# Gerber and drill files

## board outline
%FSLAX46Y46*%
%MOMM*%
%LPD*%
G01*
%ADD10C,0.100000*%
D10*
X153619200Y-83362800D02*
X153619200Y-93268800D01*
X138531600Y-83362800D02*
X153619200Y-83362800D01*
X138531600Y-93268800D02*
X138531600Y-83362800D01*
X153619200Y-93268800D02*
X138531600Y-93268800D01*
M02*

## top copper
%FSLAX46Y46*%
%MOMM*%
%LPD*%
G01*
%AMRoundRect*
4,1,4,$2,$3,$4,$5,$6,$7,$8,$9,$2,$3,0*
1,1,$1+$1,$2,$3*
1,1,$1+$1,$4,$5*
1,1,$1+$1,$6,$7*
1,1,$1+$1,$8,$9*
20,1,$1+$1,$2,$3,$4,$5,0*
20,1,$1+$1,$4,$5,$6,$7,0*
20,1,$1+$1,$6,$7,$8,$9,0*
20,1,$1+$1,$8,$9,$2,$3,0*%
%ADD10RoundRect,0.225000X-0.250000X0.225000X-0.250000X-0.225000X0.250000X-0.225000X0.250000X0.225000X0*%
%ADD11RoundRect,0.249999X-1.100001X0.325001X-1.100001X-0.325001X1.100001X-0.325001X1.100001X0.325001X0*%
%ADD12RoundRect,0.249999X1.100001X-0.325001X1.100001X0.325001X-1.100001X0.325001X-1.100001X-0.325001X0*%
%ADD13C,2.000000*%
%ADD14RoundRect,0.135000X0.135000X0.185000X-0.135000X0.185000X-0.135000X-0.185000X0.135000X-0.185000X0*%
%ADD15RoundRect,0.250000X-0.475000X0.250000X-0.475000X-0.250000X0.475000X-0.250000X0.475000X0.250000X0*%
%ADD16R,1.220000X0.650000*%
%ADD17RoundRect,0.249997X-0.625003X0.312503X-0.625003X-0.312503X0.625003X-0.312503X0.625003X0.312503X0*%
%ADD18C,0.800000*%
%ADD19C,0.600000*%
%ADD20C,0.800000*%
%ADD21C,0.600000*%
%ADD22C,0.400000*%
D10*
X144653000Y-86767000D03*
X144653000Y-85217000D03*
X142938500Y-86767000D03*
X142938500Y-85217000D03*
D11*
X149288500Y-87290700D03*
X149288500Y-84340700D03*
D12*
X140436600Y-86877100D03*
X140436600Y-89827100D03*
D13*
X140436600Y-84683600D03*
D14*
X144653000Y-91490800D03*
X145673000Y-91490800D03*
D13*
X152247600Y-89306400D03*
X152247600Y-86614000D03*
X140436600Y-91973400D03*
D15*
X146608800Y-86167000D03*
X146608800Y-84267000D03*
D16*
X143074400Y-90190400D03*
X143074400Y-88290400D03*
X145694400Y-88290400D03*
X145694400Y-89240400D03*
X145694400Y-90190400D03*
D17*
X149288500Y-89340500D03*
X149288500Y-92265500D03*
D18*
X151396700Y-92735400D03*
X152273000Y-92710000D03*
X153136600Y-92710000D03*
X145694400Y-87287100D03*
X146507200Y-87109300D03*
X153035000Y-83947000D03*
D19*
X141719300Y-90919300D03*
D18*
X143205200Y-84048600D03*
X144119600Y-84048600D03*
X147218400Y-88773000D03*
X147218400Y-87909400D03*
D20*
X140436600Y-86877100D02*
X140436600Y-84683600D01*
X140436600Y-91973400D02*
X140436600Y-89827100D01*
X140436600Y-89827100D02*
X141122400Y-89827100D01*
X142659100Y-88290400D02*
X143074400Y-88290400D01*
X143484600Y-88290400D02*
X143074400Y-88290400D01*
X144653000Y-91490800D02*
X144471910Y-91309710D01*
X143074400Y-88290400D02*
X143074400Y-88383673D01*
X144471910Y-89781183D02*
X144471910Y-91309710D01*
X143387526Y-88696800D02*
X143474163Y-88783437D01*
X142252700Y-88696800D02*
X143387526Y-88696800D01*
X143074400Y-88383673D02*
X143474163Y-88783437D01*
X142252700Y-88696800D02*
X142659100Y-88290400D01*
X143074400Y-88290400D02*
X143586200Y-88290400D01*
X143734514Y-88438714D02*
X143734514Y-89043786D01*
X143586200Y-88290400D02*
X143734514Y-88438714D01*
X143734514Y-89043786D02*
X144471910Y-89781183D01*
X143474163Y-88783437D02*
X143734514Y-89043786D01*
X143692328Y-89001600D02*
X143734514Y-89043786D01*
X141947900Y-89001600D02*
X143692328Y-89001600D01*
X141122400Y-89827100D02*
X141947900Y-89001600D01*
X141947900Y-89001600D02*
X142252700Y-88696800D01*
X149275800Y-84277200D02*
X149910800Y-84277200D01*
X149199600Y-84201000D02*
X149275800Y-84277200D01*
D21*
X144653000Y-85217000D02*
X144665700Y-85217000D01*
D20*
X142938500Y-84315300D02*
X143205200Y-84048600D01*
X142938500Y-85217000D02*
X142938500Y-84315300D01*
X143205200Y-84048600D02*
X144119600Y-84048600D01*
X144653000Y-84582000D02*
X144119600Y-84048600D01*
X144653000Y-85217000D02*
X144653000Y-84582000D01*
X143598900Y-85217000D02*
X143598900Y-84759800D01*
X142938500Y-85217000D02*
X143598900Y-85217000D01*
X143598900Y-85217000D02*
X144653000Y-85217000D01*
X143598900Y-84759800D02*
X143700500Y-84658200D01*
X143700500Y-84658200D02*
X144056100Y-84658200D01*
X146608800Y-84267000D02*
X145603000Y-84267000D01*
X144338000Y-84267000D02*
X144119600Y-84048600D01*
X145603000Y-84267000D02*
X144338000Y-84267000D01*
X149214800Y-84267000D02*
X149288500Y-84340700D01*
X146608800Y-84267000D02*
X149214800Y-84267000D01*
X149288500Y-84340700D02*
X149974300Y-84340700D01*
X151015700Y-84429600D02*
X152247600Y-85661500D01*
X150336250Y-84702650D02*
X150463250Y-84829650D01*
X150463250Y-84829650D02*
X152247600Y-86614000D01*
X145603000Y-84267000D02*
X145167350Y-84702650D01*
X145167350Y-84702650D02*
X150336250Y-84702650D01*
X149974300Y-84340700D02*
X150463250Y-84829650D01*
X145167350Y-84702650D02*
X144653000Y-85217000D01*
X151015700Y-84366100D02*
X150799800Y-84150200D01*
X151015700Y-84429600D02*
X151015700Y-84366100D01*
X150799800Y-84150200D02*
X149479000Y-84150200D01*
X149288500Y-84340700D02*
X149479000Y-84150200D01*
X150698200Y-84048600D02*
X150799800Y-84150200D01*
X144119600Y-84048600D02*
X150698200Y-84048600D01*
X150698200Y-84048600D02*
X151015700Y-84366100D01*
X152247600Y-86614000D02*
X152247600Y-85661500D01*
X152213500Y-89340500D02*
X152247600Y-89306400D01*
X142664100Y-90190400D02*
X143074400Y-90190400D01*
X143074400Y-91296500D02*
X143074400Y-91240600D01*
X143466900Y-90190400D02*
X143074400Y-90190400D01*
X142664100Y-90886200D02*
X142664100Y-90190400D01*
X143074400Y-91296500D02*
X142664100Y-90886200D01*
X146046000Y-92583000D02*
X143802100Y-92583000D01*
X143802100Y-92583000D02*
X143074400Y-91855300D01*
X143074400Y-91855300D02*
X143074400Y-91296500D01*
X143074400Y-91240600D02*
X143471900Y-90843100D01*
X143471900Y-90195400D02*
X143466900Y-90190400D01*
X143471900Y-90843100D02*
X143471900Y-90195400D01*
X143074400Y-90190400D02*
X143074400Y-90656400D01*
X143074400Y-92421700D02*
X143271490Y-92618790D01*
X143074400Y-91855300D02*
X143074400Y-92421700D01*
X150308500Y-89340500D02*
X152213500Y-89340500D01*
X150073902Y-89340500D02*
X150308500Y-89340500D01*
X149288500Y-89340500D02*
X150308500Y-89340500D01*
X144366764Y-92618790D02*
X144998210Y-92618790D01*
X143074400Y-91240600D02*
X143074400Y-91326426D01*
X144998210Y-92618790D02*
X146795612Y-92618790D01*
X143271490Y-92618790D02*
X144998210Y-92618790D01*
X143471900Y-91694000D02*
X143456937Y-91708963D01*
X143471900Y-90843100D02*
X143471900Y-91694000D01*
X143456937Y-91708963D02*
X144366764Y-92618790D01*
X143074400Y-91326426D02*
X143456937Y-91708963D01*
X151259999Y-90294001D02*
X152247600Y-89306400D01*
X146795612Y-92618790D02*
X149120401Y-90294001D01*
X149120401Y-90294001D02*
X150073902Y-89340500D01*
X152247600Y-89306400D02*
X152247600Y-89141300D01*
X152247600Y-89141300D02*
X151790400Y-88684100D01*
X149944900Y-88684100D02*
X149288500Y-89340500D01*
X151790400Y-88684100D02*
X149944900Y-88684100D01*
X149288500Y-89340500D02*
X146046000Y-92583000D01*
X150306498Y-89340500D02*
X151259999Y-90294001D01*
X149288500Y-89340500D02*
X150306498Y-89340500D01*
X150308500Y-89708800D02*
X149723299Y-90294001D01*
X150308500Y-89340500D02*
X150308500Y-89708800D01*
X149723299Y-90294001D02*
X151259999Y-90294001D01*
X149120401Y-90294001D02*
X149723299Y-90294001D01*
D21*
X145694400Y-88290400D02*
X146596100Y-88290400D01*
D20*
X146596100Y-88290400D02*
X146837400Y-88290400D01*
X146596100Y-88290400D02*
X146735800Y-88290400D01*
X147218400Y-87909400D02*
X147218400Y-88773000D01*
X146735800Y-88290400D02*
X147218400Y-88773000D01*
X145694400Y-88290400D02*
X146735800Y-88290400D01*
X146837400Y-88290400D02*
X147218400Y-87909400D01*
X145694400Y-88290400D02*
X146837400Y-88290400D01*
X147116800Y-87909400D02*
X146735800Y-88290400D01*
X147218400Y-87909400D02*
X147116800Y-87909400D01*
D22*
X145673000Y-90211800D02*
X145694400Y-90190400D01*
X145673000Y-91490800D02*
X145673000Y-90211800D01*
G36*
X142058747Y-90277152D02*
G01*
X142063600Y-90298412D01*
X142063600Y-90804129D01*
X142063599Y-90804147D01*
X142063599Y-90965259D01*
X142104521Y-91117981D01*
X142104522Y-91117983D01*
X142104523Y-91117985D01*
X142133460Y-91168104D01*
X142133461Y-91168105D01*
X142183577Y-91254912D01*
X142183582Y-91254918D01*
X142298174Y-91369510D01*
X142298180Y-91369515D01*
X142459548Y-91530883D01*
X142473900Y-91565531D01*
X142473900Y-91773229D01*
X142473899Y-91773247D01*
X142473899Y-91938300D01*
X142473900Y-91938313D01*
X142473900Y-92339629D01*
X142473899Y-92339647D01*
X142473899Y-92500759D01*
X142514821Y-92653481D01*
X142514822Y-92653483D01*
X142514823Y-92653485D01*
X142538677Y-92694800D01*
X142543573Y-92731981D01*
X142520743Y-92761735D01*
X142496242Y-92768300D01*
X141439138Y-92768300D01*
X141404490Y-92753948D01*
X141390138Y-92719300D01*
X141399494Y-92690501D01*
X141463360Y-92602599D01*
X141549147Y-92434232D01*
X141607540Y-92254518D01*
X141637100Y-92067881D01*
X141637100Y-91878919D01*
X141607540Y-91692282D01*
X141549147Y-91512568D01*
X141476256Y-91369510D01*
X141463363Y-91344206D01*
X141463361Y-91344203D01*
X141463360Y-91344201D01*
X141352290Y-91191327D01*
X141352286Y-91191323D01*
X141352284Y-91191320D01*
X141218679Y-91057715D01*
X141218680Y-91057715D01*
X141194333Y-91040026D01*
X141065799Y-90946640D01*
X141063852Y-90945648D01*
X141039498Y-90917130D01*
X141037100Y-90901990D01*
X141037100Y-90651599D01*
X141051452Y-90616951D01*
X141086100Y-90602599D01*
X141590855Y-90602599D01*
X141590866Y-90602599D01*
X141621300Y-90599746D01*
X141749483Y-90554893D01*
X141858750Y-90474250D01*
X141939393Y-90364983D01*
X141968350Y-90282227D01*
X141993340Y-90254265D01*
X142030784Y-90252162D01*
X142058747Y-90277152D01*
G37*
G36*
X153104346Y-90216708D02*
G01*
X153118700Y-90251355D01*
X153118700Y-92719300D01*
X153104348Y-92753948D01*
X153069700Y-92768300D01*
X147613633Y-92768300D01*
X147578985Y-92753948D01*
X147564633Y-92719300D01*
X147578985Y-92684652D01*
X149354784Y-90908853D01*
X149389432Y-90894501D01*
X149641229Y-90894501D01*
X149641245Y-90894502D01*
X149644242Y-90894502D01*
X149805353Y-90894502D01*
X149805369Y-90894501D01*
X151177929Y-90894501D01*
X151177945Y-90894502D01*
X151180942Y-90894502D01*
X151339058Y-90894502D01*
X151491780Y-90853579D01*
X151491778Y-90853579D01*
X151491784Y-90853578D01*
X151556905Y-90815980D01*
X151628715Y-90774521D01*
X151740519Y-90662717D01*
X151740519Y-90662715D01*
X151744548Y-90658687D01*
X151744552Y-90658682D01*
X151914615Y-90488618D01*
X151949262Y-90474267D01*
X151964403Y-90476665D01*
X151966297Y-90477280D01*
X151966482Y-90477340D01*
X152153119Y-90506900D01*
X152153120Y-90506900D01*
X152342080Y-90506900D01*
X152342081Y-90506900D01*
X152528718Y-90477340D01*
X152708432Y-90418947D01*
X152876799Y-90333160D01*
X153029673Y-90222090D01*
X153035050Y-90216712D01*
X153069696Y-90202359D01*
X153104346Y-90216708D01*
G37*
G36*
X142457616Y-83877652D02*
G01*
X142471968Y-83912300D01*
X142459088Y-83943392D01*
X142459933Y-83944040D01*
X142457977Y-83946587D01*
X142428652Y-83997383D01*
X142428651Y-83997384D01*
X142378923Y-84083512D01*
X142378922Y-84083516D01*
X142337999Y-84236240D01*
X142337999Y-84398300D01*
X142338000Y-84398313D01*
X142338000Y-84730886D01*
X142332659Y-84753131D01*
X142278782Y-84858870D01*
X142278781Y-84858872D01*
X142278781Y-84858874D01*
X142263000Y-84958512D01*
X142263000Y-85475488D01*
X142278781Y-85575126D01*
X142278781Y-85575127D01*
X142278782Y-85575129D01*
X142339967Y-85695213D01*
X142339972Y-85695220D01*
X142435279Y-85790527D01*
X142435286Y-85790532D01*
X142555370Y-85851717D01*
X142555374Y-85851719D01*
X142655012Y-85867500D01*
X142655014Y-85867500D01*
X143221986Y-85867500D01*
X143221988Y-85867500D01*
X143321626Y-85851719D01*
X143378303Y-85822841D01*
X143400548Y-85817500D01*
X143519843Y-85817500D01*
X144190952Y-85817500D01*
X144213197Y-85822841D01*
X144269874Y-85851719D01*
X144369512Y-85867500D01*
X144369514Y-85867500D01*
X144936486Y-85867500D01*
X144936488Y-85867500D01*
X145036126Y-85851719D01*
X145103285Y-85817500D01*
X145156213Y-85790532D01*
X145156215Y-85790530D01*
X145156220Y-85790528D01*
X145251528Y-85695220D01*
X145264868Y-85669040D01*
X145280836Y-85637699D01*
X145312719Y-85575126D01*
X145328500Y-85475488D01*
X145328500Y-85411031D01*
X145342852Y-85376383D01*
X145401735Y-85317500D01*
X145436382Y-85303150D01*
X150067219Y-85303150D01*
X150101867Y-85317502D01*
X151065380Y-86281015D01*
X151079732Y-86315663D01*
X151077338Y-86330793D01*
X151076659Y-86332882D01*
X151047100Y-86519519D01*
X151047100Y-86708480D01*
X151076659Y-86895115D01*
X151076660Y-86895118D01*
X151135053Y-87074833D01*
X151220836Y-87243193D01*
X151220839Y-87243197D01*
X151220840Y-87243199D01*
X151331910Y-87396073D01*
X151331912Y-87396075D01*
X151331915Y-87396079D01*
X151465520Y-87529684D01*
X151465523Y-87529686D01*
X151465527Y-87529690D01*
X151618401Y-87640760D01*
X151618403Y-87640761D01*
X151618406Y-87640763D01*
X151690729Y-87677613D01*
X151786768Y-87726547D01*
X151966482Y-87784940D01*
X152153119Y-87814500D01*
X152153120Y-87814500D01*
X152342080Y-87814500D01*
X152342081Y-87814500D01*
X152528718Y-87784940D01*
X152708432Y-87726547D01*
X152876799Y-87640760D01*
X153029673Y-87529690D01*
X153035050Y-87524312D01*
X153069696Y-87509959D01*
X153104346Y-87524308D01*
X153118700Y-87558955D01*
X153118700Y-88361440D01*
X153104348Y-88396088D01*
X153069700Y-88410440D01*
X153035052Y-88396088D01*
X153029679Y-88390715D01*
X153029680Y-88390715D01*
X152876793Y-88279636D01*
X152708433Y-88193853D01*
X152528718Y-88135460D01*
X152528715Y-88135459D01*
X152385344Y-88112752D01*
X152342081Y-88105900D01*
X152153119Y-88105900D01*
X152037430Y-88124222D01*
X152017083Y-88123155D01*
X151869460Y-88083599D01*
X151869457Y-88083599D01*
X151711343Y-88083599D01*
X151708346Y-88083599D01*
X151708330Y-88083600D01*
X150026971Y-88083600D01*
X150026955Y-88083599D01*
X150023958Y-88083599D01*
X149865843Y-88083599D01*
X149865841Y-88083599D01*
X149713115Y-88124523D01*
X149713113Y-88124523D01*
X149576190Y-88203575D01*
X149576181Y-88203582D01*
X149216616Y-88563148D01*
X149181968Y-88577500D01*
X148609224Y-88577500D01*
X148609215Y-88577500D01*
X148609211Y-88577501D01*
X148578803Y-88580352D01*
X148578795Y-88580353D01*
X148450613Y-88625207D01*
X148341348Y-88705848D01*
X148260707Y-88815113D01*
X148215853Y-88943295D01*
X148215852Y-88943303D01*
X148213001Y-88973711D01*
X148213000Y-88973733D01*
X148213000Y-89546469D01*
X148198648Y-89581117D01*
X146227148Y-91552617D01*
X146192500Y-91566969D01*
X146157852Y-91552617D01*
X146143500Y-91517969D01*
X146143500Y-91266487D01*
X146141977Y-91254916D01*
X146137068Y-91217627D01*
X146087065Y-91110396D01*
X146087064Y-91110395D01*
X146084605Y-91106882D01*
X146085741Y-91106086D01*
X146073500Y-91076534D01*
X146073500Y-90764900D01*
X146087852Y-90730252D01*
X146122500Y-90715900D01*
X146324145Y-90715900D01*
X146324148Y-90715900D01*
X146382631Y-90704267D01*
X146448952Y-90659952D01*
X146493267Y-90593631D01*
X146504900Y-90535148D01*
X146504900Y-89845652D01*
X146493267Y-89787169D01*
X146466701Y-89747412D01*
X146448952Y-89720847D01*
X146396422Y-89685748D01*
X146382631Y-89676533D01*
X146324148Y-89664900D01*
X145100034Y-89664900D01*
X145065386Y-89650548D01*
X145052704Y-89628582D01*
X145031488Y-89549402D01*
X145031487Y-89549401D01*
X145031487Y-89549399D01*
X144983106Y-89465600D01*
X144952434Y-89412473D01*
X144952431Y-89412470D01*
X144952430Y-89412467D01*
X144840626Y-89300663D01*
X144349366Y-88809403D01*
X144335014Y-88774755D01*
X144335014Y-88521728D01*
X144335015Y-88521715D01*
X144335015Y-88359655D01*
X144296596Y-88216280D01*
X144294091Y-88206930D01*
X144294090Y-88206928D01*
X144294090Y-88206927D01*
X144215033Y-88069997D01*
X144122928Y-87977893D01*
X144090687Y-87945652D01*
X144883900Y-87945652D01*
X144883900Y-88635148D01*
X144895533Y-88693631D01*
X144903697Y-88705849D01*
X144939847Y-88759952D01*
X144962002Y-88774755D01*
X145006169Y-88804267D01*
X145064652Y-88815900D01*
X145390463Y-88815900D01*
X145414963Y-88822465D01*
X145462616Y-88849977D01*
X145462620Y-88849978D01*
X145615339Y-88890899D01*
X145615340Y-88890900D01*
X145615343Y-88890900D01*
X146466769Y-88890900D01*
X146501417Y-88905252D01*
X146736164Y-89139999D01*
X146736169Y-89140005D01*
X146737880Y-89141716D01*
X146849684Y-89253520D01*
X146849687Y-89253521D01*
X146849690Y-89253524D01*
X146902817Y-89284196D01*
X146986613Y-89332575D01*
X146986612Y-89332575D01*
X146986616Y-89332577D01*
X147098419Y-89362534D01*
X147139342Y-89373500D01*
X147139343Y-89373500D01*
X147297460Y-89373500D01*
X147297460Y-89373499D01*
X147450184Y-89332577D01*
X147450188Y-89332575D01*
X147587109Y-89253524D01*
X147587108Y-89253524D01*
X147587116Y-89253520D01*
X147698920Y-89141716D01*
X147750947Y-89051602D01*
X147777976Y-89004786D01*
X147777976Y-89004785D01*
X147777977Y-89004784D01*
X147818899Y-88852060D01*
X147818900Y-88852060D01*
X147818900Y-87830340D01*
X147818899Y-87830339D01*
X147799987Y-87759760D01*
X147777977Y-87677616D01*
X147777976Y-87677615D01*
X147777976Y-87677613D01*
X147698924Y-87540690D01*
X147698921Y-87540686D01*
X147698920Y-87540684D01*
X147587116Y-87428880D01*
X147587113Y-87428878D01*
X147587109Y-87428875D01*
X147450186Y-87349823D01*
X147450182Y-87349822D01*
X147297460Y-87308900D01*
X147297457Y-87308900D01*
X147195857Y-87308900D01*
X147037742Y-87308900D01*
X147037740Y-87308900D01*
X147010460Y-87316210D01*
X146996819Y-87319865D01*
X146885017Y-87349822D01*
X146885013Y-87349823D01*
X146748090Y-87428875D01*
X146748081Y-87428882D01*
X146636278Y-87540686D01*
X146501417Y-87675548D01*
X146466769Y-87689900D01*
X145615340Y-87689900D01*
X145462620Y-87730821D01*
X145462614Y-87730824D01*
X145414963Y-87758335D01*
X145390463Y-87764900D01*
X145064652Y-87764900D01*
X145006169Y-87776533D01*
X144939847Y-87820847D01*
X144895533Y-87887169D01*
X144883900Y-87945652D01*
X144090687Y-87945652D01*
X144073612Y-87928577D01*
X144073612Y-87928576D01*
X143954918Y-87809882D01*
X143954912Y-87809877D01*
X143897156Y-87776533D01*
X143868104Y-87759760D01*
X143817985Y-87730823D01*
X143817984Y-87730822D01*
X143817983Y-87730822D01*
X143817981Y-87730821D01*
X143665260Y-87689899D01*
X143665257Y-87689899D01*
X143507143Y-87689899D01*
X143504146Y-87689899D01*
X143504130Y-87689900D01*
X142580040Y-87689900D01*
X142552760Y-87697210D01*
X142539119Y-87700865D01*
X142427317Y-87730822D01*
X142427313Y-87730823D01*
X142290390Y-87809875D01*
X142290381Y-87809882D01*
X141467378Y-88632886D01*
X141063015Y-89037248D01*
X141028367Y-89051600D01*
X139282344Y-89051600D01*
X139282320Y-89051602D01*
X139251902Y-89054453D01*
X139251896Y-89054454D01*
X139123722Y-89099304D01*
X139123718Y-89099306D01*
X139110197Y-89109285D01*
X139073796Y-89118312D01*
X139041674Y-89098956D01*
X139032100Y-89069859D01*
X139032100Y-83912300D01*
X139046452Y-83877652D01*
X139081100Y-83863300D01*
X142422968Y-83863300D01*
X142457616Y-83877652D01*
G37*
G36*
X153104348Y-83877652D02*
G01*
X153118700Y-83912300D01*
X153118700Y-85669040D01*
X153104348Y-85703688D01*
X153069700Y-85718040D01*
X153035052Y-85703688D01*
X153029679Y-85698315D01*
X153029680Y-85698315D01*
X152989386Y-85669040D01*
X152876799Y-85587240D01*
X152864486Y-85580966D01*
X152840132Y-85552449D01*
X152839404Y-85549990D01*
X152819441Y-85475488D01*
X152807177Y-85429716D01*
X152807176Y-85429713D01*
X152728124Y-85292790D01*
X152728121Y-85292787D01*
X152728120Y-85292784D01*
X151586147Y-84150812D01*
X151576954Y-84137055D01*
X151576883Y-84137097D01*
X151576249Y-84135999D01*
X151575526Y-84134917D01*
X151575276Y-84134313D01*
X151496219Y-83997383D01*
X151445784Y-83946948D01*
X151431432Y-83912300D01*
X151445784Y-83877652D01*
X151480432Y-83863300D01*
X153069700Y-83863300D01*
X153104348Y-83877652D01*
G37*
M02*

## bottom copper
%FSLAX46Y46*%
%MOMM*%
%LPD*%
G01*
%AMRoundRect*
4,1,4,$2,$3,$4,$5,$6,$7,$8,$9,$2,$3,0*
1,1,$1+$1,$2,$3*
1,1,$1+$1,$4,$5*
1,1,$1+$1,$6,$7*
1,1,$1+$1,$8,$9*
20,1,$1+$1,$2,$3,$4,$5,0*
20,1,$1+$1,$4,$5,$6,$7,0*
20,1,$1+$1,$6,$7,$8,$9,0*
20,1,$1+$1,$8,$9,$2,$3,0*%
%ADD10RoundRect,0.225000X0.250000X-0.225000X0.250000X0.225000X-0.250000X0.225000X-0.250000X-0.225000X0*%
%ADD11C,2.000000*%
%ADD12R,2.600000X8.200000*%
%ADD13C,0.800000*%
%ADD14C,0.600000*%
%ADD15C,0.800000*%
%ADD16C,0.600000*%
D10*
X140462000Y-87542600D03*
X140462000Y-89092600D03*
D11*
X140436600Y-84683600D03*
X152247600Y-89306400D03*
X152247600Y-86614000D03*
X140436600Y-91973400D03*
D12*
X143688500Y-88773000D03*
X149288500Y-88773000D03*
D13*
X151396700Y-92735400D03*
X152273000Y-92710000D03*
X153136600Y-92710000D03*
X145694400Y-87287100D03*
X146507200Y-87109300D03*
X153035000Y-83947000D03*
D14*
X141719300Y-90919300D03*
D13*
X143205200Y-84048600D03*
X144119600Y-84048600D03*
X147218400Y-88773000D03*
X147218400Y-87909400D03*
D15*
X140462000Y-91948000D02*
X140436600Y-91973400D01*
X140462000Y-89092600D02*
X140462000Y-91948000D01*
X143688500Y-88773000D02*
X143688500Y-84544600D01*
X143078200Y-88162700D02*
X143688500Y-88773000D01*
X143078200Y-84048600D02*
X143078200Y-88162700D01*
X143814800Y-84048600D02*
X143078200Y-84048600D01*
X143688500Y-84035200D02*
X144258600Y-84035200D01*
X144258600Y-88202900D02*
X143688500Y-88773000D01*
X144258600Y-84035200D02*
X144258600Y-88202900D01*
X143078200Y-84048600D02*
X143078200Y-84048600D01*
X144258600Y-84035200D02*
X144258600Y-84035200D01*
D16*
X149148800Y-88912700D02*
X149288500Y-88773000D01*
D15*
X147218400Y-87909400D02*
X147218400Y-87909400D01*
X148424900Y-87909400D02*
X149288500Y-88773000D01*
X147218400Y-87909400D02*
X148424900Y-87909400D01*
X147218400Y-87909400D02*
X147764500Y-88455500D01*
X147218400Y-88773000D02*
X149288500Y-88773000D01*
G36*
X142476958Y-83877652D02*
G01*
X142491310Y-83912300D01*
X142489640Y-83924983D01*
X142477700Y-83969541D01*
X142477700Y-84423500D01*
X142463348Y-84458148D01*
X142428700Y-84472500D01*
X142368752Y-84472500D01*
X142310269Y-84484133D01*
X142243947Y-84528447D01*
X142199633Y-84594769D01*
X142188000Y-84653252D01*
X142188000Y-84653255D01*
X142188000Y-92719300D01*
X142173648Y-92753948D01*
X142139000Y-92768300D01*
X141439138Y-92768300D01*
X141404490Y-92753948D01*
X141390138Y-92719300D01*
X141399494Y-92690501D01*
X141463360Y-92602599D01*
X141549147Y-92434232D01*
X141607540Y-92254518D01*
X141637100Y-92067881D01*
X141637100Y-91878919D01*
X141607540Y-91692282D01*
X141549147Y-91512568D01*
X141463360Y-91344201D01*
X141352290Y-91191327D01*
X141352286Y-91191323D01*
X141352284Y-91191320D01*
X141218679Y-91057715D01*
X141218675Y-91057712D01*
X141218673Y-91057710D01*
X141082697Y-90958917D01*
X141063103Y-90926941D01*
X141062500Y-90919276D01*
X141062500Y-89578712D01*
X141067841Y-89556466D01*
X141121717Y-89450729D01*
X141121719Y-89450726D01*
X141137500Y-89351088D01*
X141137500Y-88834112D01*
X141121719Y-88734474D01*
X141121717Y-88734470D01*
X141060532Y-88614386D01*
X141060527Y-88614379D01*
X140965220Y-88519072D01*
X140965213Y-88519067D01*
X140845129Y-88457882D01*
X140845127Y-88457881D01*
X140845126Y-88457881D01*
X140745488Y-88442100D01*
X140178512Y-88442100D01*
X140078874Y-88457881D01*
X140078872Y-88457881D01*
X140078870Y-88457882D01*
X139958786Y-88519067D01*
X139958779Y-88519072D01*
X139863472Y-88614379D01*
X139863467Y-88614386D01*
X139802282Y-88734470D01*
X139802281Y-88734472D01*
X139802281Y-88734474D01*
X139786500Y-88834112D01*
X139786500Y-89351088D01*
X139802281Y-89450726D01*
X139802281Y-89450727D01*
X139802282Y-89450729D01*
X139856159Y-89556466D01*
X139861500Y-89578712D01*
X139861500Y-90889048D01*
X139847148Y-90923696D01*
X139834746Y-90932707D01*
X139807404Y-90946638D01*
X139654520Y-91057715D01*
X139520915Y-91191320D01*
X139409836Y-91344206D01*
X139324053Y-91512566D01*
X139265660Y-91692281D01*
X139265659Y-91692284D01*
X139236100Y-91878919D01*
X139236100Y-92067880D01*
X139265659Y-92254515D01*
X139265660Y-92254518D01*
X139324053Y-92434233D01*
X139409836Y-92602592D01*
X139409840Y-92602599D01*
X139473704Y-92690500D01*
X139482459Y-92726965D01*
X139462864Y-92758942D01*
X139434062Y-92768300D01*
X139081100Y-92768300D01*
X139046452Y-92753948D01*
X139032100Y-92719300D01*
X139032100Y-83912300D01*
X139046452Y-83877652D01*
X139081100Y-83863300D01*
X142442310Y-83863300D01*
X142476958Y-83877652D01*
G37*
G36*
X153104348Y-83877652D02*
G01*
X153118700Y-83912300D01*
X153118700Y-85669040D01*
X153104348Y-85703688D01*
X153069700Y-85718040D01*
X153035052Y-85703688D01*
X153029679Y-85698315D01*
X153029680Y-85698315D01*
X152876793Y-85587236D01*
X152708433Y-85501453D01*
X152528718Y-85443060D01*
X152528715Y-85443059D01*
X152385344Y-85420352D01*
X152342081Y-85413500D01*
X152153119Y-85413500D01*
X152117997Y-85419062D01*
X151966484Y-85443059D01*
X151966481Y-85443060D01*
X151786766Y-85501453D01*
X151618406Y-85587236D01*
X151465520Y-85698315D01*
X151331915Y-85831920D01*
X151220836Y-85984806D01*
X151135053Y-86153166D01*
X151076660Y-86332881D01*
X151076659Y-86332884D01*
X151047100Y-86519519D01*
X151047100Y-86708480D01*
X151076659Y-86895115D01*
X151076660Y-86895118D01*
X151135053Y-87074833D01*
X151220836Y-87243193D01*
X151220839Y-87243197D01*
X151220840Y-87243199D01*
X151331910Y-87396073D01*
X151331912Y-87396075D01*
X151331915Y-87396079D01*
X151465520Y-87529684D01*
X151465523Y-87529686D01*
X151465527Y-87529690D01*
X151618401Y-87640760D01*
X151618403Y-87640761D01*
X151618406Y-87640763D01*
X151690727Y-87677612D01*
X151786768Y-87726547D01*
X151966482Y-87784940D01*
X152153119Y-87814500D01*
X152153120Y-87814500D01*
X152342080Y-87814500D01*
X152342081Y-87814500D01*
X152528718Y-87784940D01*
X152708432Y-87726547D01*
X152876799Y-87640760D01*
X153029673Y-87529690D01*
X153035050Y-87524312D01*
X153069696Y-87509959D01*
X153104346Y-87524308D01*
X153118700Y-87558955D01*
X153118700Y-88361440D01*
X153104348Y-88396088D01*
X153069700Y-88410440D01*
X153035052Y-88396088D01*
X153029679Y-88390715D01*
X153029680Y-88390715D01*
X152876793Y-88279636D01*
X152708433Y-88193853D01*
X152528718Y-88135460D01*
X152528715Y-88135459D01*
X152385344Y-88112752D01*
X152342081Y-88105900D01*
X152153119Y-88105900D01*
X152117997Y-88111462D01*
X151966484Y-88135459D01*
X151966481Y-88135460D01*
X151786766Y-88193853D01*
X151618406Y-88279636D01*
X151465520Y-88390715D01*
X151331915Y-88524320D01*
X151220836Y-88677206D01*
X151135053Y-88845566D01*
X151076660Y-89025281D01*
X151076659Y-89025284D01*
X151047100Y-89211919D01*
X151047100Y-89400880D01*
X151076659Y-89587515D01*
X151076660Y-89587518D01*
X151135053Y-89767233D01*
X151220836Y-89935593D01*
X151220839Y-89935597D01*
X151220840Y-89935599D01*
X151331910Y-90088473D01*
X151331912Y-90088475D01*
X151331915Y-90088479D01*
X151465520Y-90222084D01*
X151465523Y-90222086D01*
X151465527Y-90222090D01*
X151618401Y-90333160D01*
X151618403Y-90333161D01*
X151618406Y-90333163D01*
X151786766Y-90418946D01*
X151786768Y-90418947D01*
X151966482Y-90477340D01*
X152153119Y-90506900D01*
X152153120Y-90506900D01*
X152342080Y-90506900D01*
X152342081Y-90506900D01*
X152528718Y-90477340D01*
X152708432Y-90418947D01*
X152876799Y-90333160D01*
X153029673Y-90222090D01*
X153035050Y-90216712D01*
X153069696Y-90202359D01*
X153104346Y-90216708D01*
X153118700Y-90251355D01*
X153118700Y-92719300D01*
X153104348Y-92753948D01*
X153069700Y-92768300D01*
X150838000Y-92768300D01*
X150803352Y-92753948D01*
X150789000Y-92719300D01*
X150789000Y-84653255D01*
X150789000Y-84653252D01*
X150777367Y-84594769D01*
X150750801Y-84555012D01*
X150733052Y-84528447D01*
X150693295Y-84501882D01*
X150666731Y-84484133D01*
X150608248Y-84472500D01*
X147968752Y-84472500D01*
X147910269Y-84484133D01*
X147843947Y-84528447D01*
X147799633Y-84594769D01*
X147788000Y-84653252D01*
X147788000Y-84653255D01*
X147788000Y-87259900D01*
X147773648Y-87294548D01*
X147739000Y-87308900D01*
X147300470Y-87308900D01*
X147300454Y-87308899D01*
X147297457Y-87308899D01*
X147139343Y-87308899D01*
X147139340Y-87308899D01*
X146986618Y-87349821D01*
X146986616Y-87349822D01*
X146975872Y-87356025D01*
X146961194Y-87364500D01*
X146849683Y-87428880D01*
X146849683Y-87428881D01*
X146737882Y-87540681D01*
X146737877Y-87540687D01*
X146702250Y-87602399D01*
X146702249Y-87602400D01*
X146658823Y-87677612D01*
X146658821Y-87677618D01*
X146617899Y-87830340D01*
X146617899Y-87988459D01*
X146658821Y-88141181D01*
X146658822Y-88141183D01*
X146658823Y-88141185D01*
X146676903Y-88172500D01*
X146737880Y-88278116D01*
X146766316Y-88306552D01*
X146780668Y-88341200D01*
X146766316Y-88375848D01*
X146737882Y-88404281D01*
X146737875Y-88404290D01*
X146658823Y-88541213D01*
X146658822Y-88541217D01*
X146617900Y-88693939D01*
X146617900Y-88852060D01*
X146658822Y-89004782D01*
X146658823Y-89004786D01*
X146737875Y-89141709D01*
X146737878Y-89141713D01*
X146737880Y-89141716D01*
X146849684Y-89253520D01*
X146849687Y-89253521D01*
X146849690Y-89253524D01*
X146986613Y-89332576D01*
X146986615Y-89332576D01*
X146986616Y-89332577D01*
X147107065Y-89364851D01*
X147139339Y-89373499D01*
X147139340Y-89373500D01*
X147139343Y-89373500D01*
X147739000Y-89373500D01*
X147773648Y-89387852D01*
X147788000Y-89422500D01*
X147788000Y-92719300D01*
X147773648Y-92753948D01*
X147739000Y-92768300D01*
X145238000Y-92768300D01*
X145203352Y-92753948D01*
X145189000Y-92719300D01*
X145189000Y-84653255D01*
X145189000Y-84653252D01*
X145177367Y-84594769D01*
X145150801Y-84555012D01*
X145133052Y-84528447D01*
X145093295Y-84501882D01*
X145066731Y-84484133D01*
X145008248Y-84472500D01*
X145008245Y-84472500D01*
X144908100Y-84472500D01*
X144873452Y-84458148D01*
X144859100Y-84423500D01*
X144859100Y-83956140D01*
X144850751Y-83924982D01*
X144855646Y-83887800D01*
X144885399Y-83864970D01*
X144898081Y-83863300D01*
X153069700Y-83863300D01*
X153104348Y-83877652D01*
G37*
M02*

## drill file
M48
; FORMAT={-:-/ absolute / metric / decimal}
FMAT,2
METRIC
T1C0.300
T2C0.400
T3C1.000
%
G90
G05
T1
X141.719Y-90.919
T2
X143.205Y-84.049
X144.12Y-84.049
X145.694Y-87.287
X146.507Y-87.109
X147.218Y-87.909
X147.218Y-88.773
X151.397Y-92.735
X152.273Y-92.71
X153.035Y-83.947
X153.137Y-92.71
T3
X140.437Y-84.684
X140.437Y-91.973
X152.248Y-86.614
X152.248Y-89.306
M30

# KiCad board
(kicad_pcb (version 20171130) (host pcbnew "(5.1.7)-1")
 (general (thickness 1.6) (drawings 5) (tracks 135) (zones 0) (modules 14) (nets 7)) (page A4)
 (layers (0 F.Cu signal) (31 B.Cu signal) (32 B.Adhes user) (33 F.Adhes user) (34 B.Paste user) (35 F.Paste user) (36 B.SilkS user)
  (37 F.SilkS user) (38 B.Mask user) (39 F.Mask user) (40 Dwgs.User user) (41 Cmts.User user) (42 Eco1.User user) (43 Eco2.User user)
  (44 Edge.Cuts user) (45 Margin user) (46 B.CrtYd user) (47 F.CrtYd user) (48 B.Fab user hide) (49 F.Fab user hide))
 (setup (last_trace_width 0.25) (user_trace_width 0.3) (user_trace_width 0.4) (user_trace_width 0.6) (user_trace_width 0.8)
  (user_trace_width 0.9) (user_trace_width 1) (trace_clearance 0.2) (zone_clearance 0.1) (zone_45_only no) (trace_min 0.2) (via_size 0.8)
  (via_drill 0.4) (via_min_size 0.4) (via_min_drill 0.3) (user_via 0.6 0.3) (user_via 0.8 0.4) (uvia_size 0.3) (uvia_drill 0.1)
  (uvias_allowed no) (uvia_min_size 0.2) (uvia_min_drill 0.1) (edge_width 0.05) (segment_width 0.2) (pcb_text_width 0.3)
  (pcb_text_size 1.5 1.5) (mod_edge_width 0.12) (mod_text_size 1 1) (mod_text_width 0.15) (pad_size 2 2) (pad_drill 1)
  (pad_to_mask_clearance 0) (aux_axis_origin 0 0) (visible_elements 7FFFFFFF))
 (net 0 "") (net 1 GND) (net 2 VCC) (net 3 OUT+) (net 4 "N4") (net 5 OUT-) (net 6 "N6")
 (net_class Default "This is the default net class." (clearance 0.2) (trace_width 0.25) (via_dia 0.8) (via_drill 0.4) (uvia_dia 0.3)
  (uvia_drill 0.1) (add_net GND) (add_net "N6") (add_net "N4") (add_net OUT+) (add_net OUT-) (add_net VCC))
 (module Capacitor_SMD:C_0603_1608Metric (layer B.Cu) (at 140.462 88.3176 90)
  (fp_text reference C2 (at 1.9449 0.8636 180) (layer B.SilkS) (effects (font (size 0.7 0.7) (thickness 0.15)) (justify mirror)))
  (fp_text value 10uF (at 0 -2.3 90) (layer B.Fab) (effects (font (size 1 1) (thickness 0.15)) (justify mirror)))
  (pad 2 smd roundrect (at 0.775 0 90) (size 0.9 0.95) (layers B.Cu B.Paste B.Mask) (roundrect_rratio 0.25) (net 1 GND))
  (pad 1 smd roundrect (at -0.775 0 90) (size 0.9 0.95) (layers B.Cu B.Paste B.Mask) (roundrect_rratio 0.25) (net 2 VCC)))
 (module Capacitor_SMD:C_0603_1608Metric (layer F.Cu) (at 144.653 85.992 270)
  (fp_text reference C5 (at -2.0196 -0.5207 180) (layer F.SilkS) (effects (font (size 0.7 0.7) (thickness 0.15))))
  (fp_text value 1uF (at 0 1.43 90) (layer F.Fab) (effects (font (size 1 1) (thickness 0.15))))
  (pad 2 smd roundrect (at 0.775 0 270) (size 0.9 0.95) (layers F.Cu F.Paste F.Mask) (roundrect_rratio 0.25) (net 1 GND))
  (pad 1 smd roundrect (at -0.775 0 270) (size 0.9 0.95) (layers F.Cu F.Paste F.Mask) (roundrect_rratio 0.25) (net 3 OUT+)))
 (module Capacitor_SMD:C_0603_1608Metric (layer F.Cu) (at 142.9385 85.992 270)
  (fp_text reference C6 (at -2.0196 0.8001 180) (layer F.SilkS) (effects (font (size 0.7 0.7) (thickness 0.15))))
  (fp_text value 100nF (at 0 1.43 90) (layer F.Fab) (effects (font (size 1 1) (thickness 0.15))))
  (pad 2 smd roundrect (at 0.775 0 270) (size 0.9 0.95) (layers F.Cu F.Paste F.Mask) (roundrect_rratio 0.25) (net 1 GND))
  (pad 1 smd roundrect (at -0.775 0 270) (size 0.9 0.95) (layers F.Cu F.Paste F.Mask) (roundrect_rratio 0.25) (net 3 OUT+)))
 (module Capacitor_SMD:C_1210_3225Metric (layer F.Cu) (at 149.2885 85.8157 270)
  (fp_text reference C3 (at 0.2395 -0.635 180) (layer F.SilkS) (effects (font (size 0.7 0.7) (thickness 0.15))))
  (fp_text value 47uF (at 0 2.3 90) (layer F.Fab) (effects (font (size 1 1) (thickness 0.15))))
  (pad 2 smd roundrect (at 1.475 0 270) (size 1.15 2.7) (layers F.Cu F.Paste F.Mask) (roundrect_rratio 0.2173904347826087) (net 1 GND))
  (pad 1 smd roundrect (at -1.475 0 270) (size 1.15 2.7) (layers F.Cu F.Paste F.Mask) (roundrect_rratio 0.2173904347826087) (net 3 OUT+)))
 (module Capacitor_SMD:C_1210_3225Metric (layer F.Cu) (at 140.4366 88.3521 90)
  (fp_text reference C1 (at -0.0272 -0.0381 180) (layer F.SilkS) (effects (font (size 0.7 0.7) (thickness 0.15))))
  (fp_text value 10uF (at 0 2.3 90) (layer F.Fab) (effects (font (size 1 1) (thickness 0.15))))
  (pad 2 smd roundrect (at 1.475 0 90) (size 1.15 2.7) (layers F.Cu F.Paste F.Mask) (roundrect_rratio 0.2173904347826087) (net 1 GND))
  (pad 1 smd roundrect (at -1.475 0 90) (size 1.15 2.7) (layers F.Cu F.Paste F.Mask) (roundrect_rratio 0.2173904347826087) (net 2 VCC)))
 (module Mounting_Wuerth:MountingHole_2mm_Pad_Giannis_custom (layer F.Cu) (at 140.4366 84.3661)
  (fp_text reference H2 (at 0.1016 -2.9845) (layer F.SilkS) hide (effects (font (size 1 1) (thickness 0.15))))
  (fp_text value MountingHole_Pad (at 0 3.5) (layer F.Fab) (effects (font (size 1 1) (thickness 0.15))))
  (pad 1 thru_hole circle (at 0 0.3175) (size 2 2) (drill 1) (layers *.Cu *.Mask) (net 1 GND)))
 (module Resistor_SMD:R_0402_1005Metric (layer F.Cu) (at 145.163 91.4908 180)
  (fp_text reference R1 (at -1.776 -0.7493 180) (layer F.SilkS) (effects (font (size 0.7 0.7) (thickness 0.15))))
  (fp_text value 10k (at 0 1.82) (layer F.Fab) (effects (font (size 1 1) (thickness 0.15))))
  (pad 2 smd roundrect (at 0.51 0 180) (size 0.54 0.64) (layers F.Cu F.Paste F.Mask) (roundrect_rratio 0.25) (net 2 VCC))
  (pad 1 smd roundrect (at -0.51 0 180) (size 0.54 0.64) (layers F.Cu F.Paste F.Mask) (roundrect_rratio 0.25) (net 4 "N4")))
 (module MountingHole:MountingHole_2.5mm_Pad (layer F.Cu) (at 154.686 89.408)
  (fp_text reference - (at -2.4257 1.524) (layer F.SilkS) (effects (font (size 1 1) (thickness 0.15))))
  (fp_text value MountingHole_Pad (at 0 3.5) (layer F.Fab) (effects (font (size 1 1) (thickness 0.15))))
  (pad 1 thru_hole circle (at -2.4384 -0.1016) (size 2 2) (drill 1) (layers *.Cu *.Mask) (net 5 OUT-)))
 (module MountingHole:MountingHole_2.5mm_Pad (layer F.Cu) (at 154.686 86.106)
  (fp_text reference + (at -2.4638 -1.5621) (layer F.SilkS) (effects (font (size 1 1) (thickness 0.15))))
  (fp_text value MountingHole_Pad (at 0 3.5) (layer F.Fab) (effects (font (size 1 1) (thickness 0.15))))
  (pad 1 thru_hole circle (at -2.4384 0.508) (size 2 2) (drill 1) (layers *.Cu *.Mask) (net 3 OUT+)))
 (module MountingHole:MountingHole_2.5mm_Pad (layer F.Cu) (at 139.6746 89.8271)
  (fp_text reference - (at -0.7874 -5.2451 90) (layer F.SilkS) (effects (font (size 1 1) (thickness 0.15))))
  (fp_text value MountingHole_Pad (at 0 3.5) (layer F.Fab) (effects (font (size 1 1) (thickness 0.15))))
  (pad 1 thru_hole circle (at 0.762 2.1463) (size 2 2) (drill 1) (layers *.Cu *.Mask) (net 2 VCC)))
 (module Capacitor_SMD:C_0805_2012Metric (layer F.Cu) (at 146.6088 85.217 270)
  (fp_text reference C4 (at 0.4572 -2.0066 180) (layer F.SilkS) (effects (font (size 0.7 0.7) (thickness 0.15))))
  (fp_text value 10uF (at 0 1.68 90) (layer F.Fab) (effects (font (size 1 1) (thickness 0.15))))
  (pad 2 smd roundrect (at 0.95 0 270) (size 1 1.45) (layers F.Cu F.Paste F.Mask) (roundrect_rratio 0.25) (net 1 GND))
  (pad 1 smd roundrect (at -0.95 0 270) (size 1 1.45) (layers F.Cu F.Paste F.Mask) (roundrect_rratio 0.25) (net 3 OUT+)))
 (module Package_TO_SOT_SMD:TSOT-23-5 (layer F.Cu) (at 144.3844 89.2404 180)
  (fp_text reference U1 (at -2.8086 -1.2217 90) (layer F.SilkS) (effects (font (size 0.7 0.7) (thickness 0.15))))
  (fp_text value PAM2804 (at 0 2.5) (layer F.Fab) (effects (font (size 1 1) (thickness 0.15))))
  (pad 5 smd rect (at 1.31 -0.95 180) (size 1.22 0.65) (layers F.Cu F.Paste F.Mask) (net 5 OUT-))
  (pad 4 smd rect (at 1.31 0.95 180) (size 1.22 0.65) (layers F.Cu F.Paste F.Mask) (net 2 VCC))
  (pad 3 smd rect (at -1.31 0.95 180) (size 1.22 0.65) (layers F.Cu F.Paste F.Mask) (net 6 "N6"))
  (pad 2 smd rect (at -1.31 0 180) (size 1.22 0.65) (layers F.Cu F.Paste F.Mask) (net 1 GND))
  (pad 1 smd rect (at -1.31 -0.95 180) (size 1.22 0.65) (layers F.Cu F.Paste F.Mask) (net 4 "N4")))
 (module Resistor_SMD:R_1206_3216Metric (layer F.Cu) (at 149.2885 90.803 270)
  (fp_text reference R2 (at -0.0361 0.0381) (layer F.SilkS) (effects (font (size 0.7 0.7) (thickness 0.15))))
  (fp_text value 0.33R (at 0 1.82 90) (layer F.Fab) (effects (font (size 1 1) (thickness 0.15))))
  (pad 1 smd roundrect (at -1.4625 0 270) (size 1.125 1.75) (layers F.Cu F.Paste F.Mask) (roundrect_rratio 0.2222195555555556) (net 5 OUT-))
  (pad 2 smd roundrect (at 1.4625 0 270) (size 1.125 1.75) (layers F.Cu F.Paste F.Mask) (roundrect_rratio 0.2222195555555556) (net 1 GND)))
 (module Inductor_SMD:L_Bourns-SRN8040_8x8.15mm (layer B.Cu) (at 146.4885 88.773 180)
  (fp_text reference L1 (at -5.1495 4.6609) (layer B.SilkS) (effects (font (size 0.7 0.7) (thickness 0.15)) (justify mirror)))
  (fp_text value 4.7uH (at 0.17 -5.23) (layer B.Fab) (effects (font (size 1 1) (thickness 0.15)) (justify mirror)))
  (pad 2 smd rect (at 2.8 0 180) (size 2.6 8.2) (layers B.Cu B.Paste B.Mask) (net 3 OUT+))
  (pad 1 smd rect (at -2.8 0 180) (size 2.6 8.2) (layers B.Cu B.Paste B.Mask) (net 6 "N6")))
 (gr_line (start 153.6192 83.3628) (end 153.6192 93.2688) (layer Edge.Cuts) (width 0.1))
 (gr_line (start 138.5316 83.3628) (end 153.6192 83.3628) (layer Edge.Cuts) (width 0.1))
 (gr_line (start 138.5316 93.2688) (end 138.5316 83.3628) (layer Edge.Cuts) (width 0.1))
 (gr_line (start 153.6192 93.2688) (end 138.5316 93.2688) (layer Edge.Cuts) (width 0.1))
 (segment (start 140.4366 86.8771) (end 140.4366 84.6836) (width 0.8) (layer F.Cu) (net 1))
 (via (at 151.3967 92.7354) (size 0.8) (drill 0.4) (layers F.Cu B.Cu) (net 1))
 (via (at 152.273 92.71) (size 0.8) (drill 0.4) (layers F.Cu B.Cu) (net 1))
 (via (at 153.1366 92.71) (size 0.8) (drill 0.4) (layers F.Cu B.Cu) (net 1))
 (via (at 145.6944 87.2871) (size 0.8) (drill 0.4) (layers F.Cu B.Cu) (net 1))
 (via (at 146.5072 87.1093) (size 0.8) (drill 0.4) (layers F.Cu B.Cu) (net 1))
 (via (at 153.035 83.947) (size 0.8) (drill 0.4) (layers F.Cu B.Cu) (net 1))
 (via (at 141.7193 90.9193) (size 0.6) (drill 0.3) (layers F.Cu B.Cu) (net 1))
 (segment (start 140.4366 91.9734) (end 140.4366 89.8271) (width 0.8) (layer F.Cu) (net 2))
 (segment (start 140.4366 89.8271) (end 141.1224 89.8271) (width 0.8) (layer F.Cu) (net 2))
 (segment (start 142.6591 88.2904) (end 143.0744 88.2904) (width 0.8) (layer F.Cu) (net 2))
 (segment (start 143.4846 88.2904) (end 143.0744 88.2904) (width 0.8) (layer F.Cu) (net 2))
 (segment (start 144.653 91.4908) (end 144.47191 91.30971) (width 0.8) (layer F.Cu) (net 2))
 (segment (start 143.0744 88.2904) (end 143.0744 88.383673) (width 0.8) (layer F.Cu) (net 2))
 (segment (start 144.47191 89.781183) (end 144.47191 91.30971) (width 0.8) (layer F.Cu) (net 2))
 (segment (start 143.387526 88.6968) (end 143.474163 88.783437) (width 0.8) (layer F.Cu) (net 2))
 (segment (start 142.2527 88.6968) (end 143.387526 88.6968) (width 0.8) (layer F.Cu) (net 2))
 (segment (start 143.0744 88.383673) (end 143.474163 88.783437) (width 0.8) (layer F.Cu) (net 2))
 (segment (start 142.2527 88.6968) (end 142.6591 88.2904) (width 0.8) (layer F.Cu) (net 2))
 (segment (start 143.0744 88.2904) (end 143.5862 88.2904) (width 0.8) (layer F.Cu) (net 2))
 (segment (start 143.734514 88.438714) (end 143.734514 89.043786) (width 0.8) (layer F.Cu) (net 2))
 (segment (start 143.5862 88.2904) (end 143.734514 88.438714) (width 0.8) (layer F.Cu) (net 2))
 (segment (start 143.734514 89.043786) (end 144.47191 89.781183) (width 0.8) (layer F.Cu) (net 2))
 (segment (start 143.474163 88.783437) (end 143.734514 89.043786) (width 0.8) (layer F.Cu) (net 2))
 (segment (start 143.692328 89.0016) (end 143.734514 89.043786) (width 0.8) (layer F.Cu) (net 2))
 (segment (start 141.9479 89.0016) (end 143.692328 89.0016) (width 0.8) (layer F.Cu) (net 2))
 (segment (start 141.1224 89.8271) (end 141.9479 89.0016) (width 0.8) (layer F.Cu) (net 2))
 (segment (start 141.9479 89.0016) (end 142.2527 88.6968) (width 0.8) (layer F.Cu) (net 2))
 (segment (start 140.462 91.948) (end 140.4366 91.9734) (width 0.8) (layer B.Cu) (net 2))
 (segment (start 140.462 89.0926) (end 140.462 91.948) (width 0.8) (layer B.Cu) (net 2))
 (segment (start 149.2758 84.2772) (end 149.9108 84.2772) (width 0.8) (layer F.Cu) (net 3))
 (segment (start 149.1996 84.201) (end 149.2758 84.2772) (width 0.8) (layer F.Cu) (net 3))
 (segment (start 144.653 85.217) (end 144.6657 85.217) (width 0.6) (layer F.Cu) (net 3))
 (segment (start 143.6885 88.773) (end 143.6885 84.5446) (width 0.8) (layer B.Cu) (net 3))
 (segment (start 143.0782 88.1627) (end 143.6885 88.773) (width 0.8) (layer B.Cu) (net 3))
 (segment (start 143.0782 84.0486) (end 143.0782 88.1627) (width 0.8) (layer B.Cu) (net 3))
 (segment (start 143.8148 84.0486) (end 143.0782 84.0486) (width 0.8) (layer B.Cu) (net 3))
 (segment (start 143.6885 84.0352) (end 144.2586 84.0352) (width 0.8) (layer B.Cu) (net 3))
 (segment (start 144.2586 88.2029) (end 143.6885 88.773) (width 0.8) (layer B.Cu) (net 3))
 (segment (start 144.2586 84.0352) (end 144.2586 88.2029) (width 0.8) (layer B.Cu) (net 3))
 (segment (start 143.0782 84.0486) (end 143.0782 84.0486) (width 0.8) (layer B.Cu) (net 3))
 (via (at 143.2052 84.0486) (size 0.8) (drill 0.4) (layers F.Cu B.Cu) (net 3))
 (segment (start 144.2586 84.0352) (end 144.2586 84.0352) (width 0.8) (layer B.Cu) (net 3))
 (via (at 144.1196 84.0486) (size 0.8) (drill 0.4) (layers F.Cu B.Cu) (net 3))
 (segment (start 142.9385 84.3153) (end 143.2052 84.0486) (width 0.8) (layer F.Cu) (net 3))
 (segment (start 142.9385 85.217) (end 142.9385 84.3153) (width 0.8) (layer F.Cu) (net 3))
 (segment (start 143.2052 84.0486) (end 144.1196 84.0486) (width 0.8) (layer F.Cu) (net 3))
 (segment (start 144.653 84.582) (end 144.1196 84.0486) (width 0.8) (layer F.Cu) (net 3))
 (segment (start 144.653 85.217) (end 144.653 84.582) (width 0.8) (layer F.Cu) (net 3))
 (segment (start 143.5989 85.217) (end 143.5989 84.7598) (width 0.8) (layer F.Cu) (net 3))
 (segment (start 142.9385 85.217) (end 143.5989 85.217) (width 0.8) (layer F.Cu) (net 3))
 (segment (start 143.5989 85.217) (end 144.653 85.217) (width 0.8) (layer F.Cu) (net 3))
 (segment (start 143.5989 84.7598) (end 143.7005 84.6582) (width 0.8) (layer F.Cu) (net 3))
 (segment (start 143.7005 84.6582) (end 144.0561 84.6582) (width 0.8) (layer F.Cu) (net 3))
 (segment (start 146.6088 84.267) (end 145.603 84.267) (width 0.8) (layer F.Cu) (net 3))
 (segment (start 144.338 84.267) (end 144.1196 84.0486) (width 0.8) (layer F.Cu) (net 3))
 (segment (start 145.603 84.267) (end 144.338 84.267) (width 0.8) (layer F.Cu) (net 3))
 (segment (start 149.2148 84.267) (end 149.2885 84.3407) (width 0.8) (layer F.Cu) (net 3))
 (segment (start 146.6088 84.267) (end 149.2148 84.267) (width 0.8) (layer F.Cu) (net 3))
 (segment (start 149.2885 84.3407) (end 149.9743 84.3407) (width 0.8) (layer F.Cu) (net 3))
 (segment (start 151.0157 84.4296) (end 152.2476 85.6615) (width 0.8) (layer F.Cu) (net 3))
 (segment (start 150.33625 84.70265) (end 150.46325 84.82965) (width 0.8) (layer F.Cu) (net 3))
 (segment (start 150.46325 84.82965) (end 152.2476 86.614) (width 0.8) (layer F.Cu) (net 3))
 (segment (start 145.603 84.267) (end 145.16735 84.70265) (width 0.8) (layer F.Cu) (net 3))
 (segment (start 145.16735 84.70265) (end 150.33625 84.70265) (width 0.8) (layer F.Cu) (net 3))
 (segment (start 149.9743 84.3407) (end 150.46325 84.82965) (width 0.8) (layer F.Cu) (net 3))
 (segment (start 145.16735 84.70265) (end 144.653 85.217) (width 0.8) (layer F.Cu) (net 3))
 (segment (start 151.0157 84.3661) (end 150.7998 84.1502) (width 0.8) (layer F.Cu) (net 3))
 (segment (start 151.0157 84.4296) (end 151.0157 84.3661) (width 0.8) (layer F.Cu) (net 3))
 (segment (start 150.7998 84.1502) (end 149.479 84.1502) (width 0.8) (layer F.Cu) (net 3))
 (segment (start 149.2885 84.3407) (end 149.479 84.1502) (width 0.8) (layer F.Cu) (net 3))
 (segment (start 150.6982 84.0486) (end 150.7998 84.1502) (width 0.8) (layer F.Cu) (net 3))
 (segment (start 144.1196 84.0486) (end 150.6982 84.0486) (width 0.8) (layer F.Cu) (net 3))
 (segment (start 150.6982 84.0486) (end 151.0157 84.3661) (width 0.8) (layer F.Cu) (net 3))
 (segment (start 152.2476 86.614) (end 152.2476 85.6615) (width 0.8) (layer F.Cu) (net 3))
 (segment (start 152.2135 89.3405) (end 152.2476 89.3064) (width 0.8) (layer F.Cu) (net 5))
 (segment (start 142.6641 90.1904) (end 143.0744 90.1904) (width 0.8) (layer F.Cu) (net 5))
 (segment (start 143.0744 91.2965) (end 143.0744 91.2406) (width 0.8) (layer F.Cu) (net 5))
 (segment (start 143.4669 90.1904) (end 143.0744 90.1904) (width 0.8) (layer F.Cu) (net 5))
 (segment (start 142.6641 90.8862) (end 142.6641 90.1904) (width 0.8) (layer F.Cu) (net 5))
 (segment (start 143.0744 91.2965) (end 142.6641 90.8862) (width 0.8) (layer F.Cu) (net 5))
 (segment (start 146.046 92.583) (end 143.8021 92.583) (width 0.8) (layer F.Cu) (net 5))
 (segment (start 143.8021 92.583) (end 143.0744 91.8553) (width 0.8) (layer F.Cu) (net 5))
 (segment (start 143.0744 91.8553) (end 143.0744 91.2965) (width 0.8) (layer F.Cu) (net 5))
 (segment (start 143.0744 91.2406) (end 143.4719 90.8431) (width 0.8) (layer F.Cu) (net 5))
 (segment (start 143.4719 90.1954) (end 143.4669 90.1904) (width 0.8) (layer F.Cu) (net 5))
 (segment (start 143.4719 90.8431) (end 143.4719 90.1954) (width 0.8) (layer F.Cu) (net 5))
 (segment (start 143.0744 90.1904) (end 143.0744 90.6564) (width 0.8) (layer F.Cu) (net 5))
 (segment (start 143.0744 92.4217) (end 143.27149 92.61879) (width 0.8) (layer F.Cu) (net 5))
 (segment (start 143.0744 91.8553) (end 143.0744 92.4217) (width 0.8) (layer F.Cu) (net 5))
 (segment (start 150.3085 89.3405) (end 152.2135 89.3405) (width 0.8) (layer F.Cu) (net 5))
 (segment (start 150.073902 89.3405) (end 150.3085 89.3405) (width 0.8) (layer F.Cu) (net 5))
 (segment (start 149.2885 89.3405) (end 150.3085 89.3405) (width 0.8) (layer F.Cu) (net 5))
 (segment (start 144.366764 92.61879) (end 144.99821 92.61879) (width 0.8) (layer F.Cu) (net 5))
 (segment (start 143.0744 91.2406) (end 143.0744 91.326426) (width 0.8) (layer F.Cu) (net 5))
 (segment (start 144.99821 92.61879) (end 146.795612 92.61879) (width 0.8) (layer F.Cu) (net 5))
 (segment (start 143.27149 92.61879) (end 144.99821 92.61879) (width 0.8) (layer F.Cu) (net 5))
 (segment (start 143.4719 91.694) (end 143.456937 91.708963) (width 0.8) (layer F.Cu) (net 5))
 (segment (start 143.4719 90.8431) (end 143.4719 91.694) (width 0.8) (layer F.Cu) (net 5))
 (segment (start 143.456937 91.708963) (end 144.366764 92.61879) (width 0.8) (layer F.Cu) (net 5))
 (segment (start 143.0744 91.326426) (end 143.456937 91.708963) (width 0.8) (layer F.Cu) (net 5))
 (segment (start 151.259999 90.294001) (end 152.2476 89.3064) (width 0.8) (layer F.Cu) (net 5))
 (segment (start 146.795612 92.61879) (end 149.120401 90.294001) (width 0.8) (layer F.Cu) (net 5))
 (segment (start 149.120401 90.294001) (end 150.073902 89.3405) (width 0.8) (layer F.Cu) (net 5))
 (segment (start 152.2476 89.3064) (end 152.2476 89.1413) (width 0.8) (layer F.Cu) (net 5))
 (segment (start 152.2476 89.1413) (end 151.7904 88.6841) (width 0.8) (layer F.Cu) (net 5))
 (segment (start 149.9449 88.6841) (end 149.2885 89.3405) (width 0.8) (layer F.Cu) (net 5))
 (segment (start 151.7904 88.6841) (end 149.9449 88.6841) (width 0.8) (layer F.Cu) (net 5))
 (segment (start 149.2885 89.3405) (end 146.046 92.583) (width 0.8) (layer F.Cu) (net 5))
 (segment (start 150.306498 89.3405) (end 151.259999 90.294001) (width 0.8) (layer F.Cu) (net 5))
 (segment (start 149.2885 89.3405) (end 150.306498 89.3405) (width 0.8) (layer F.Cu) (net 5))
 (segment (start 150.3085 89.7088) (end 149.723299 90.294001) (width 0.8) (layer F.Cu) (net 5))
 (segment (start 150.3085 89.3405) (end 150.3085 89.7088) (width 0.8) (layer F.Cu) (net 5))
 (segment (start 149.723299 90.294001) (end 151.259999 90.294001) (width 0.8) (layer F.Cu) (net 5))
 (segment (start 149.120401 90.294001) (end 149.723299 90.294001) (width 0.8) (layer F.Cu) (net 5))
 (via (at 147.2184 88.773) (size 0.8) (drill 0.4) (layers F.Cu B.Cu) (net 6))
 (segment (start 149.1488 88.9127) (end 149.2885 88.773) (width 0.6) (layer B.Cu) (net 6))
 (segment (start 145.6944 88.2904) (end 146.5961 88.2904) (width 0.6) (layer F.Cu) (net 6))
 (segment (start 147.2184 87.9094) (end 147.2184 87.9094) (width 0.8) (layer B.Cu) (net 6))
 (via (at 147.2184 87.9094) (size 0.8) (drill 0.4) (layers F.Cu B.Cu) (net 6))
 (segment (start 148.4249 87.9094) (end 149.2885 88.773) (width 0.8) (layer B.Cu) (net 6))
 (segment (start 147.2184 87.9094) (end 148.4249 87.9094) (width 0.8) (layer B.Cu) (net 6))
 (segment (start 147.2184 87.9094) (end 147.7645 88.4555) (width 0.8) (layer B.Cu) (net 6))
 (segment (start 147.2184 88.773) (end 149.2885 88.773) (width 0.8) (layer B.Cu) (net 6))
 (segment (start 146.5961 88.2904) (end 146.8374 88.2904) (width 0.8) (layer F.Cu) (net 6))
 (segment (start 146.5961 88.2904) (end 146.7358 88.2904) (width 0.8) (layer F.Cu) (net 6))
 (segment (start 147.2184 87.9094) (end 147.2184 88.773) (width 0.8) (layer F.Cu) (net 6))
 (segment (start 146.7358 88.2904) (end 147.2184 88.773) (width 0.8) (layer F.Cu) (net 6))
 (segment (start 145.6944 88.2904) (end 146.7358 88.2904) (width 0.8) (layer F.Cu) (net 6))
 (segment (start 146.8374 88.2904) (end 147.2184 87.9094) (width 0.8) (layer F.Cu) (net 6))
 (segment (start 145.6944 88.2904) (end 146.8374 88.2904) (width 0.8) (layer F.Cu) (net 6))
 (segment (start 147.1168 87.9094) (end 146.7358 88.2904) (width 0.8) (layer F.Cu) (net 6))
 (segment (start 147.2184 87.9094) (end 147.1168 87.9094) (width 0.8) (layer F.Cu) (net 6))
 (segment (start 145.673 90.2118) (end 145.6944 90.1904) (width 0.4) (layer F.Cu) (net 4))
 (segment (start 145.673 91.4908) (end 145.673 90.2118) (width 0.4) (layer F.Cu) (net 4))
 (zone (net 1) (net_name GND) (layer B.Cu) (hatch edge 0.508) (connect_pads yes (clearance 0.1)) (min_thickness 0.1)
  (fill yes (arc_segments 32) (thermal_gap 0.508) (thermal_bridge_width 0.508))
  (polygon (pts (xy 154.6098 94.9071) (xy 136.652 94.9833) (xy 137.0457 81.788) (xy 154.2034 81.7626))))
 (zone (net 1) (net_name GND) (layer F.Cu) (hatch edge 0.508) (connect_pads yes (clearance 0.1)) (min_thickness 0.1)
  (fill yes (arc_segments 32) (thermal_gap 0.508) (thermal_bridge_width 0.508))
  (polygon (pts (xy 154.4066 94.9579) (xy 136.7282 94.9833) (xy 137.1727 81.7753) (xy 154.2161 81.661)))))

